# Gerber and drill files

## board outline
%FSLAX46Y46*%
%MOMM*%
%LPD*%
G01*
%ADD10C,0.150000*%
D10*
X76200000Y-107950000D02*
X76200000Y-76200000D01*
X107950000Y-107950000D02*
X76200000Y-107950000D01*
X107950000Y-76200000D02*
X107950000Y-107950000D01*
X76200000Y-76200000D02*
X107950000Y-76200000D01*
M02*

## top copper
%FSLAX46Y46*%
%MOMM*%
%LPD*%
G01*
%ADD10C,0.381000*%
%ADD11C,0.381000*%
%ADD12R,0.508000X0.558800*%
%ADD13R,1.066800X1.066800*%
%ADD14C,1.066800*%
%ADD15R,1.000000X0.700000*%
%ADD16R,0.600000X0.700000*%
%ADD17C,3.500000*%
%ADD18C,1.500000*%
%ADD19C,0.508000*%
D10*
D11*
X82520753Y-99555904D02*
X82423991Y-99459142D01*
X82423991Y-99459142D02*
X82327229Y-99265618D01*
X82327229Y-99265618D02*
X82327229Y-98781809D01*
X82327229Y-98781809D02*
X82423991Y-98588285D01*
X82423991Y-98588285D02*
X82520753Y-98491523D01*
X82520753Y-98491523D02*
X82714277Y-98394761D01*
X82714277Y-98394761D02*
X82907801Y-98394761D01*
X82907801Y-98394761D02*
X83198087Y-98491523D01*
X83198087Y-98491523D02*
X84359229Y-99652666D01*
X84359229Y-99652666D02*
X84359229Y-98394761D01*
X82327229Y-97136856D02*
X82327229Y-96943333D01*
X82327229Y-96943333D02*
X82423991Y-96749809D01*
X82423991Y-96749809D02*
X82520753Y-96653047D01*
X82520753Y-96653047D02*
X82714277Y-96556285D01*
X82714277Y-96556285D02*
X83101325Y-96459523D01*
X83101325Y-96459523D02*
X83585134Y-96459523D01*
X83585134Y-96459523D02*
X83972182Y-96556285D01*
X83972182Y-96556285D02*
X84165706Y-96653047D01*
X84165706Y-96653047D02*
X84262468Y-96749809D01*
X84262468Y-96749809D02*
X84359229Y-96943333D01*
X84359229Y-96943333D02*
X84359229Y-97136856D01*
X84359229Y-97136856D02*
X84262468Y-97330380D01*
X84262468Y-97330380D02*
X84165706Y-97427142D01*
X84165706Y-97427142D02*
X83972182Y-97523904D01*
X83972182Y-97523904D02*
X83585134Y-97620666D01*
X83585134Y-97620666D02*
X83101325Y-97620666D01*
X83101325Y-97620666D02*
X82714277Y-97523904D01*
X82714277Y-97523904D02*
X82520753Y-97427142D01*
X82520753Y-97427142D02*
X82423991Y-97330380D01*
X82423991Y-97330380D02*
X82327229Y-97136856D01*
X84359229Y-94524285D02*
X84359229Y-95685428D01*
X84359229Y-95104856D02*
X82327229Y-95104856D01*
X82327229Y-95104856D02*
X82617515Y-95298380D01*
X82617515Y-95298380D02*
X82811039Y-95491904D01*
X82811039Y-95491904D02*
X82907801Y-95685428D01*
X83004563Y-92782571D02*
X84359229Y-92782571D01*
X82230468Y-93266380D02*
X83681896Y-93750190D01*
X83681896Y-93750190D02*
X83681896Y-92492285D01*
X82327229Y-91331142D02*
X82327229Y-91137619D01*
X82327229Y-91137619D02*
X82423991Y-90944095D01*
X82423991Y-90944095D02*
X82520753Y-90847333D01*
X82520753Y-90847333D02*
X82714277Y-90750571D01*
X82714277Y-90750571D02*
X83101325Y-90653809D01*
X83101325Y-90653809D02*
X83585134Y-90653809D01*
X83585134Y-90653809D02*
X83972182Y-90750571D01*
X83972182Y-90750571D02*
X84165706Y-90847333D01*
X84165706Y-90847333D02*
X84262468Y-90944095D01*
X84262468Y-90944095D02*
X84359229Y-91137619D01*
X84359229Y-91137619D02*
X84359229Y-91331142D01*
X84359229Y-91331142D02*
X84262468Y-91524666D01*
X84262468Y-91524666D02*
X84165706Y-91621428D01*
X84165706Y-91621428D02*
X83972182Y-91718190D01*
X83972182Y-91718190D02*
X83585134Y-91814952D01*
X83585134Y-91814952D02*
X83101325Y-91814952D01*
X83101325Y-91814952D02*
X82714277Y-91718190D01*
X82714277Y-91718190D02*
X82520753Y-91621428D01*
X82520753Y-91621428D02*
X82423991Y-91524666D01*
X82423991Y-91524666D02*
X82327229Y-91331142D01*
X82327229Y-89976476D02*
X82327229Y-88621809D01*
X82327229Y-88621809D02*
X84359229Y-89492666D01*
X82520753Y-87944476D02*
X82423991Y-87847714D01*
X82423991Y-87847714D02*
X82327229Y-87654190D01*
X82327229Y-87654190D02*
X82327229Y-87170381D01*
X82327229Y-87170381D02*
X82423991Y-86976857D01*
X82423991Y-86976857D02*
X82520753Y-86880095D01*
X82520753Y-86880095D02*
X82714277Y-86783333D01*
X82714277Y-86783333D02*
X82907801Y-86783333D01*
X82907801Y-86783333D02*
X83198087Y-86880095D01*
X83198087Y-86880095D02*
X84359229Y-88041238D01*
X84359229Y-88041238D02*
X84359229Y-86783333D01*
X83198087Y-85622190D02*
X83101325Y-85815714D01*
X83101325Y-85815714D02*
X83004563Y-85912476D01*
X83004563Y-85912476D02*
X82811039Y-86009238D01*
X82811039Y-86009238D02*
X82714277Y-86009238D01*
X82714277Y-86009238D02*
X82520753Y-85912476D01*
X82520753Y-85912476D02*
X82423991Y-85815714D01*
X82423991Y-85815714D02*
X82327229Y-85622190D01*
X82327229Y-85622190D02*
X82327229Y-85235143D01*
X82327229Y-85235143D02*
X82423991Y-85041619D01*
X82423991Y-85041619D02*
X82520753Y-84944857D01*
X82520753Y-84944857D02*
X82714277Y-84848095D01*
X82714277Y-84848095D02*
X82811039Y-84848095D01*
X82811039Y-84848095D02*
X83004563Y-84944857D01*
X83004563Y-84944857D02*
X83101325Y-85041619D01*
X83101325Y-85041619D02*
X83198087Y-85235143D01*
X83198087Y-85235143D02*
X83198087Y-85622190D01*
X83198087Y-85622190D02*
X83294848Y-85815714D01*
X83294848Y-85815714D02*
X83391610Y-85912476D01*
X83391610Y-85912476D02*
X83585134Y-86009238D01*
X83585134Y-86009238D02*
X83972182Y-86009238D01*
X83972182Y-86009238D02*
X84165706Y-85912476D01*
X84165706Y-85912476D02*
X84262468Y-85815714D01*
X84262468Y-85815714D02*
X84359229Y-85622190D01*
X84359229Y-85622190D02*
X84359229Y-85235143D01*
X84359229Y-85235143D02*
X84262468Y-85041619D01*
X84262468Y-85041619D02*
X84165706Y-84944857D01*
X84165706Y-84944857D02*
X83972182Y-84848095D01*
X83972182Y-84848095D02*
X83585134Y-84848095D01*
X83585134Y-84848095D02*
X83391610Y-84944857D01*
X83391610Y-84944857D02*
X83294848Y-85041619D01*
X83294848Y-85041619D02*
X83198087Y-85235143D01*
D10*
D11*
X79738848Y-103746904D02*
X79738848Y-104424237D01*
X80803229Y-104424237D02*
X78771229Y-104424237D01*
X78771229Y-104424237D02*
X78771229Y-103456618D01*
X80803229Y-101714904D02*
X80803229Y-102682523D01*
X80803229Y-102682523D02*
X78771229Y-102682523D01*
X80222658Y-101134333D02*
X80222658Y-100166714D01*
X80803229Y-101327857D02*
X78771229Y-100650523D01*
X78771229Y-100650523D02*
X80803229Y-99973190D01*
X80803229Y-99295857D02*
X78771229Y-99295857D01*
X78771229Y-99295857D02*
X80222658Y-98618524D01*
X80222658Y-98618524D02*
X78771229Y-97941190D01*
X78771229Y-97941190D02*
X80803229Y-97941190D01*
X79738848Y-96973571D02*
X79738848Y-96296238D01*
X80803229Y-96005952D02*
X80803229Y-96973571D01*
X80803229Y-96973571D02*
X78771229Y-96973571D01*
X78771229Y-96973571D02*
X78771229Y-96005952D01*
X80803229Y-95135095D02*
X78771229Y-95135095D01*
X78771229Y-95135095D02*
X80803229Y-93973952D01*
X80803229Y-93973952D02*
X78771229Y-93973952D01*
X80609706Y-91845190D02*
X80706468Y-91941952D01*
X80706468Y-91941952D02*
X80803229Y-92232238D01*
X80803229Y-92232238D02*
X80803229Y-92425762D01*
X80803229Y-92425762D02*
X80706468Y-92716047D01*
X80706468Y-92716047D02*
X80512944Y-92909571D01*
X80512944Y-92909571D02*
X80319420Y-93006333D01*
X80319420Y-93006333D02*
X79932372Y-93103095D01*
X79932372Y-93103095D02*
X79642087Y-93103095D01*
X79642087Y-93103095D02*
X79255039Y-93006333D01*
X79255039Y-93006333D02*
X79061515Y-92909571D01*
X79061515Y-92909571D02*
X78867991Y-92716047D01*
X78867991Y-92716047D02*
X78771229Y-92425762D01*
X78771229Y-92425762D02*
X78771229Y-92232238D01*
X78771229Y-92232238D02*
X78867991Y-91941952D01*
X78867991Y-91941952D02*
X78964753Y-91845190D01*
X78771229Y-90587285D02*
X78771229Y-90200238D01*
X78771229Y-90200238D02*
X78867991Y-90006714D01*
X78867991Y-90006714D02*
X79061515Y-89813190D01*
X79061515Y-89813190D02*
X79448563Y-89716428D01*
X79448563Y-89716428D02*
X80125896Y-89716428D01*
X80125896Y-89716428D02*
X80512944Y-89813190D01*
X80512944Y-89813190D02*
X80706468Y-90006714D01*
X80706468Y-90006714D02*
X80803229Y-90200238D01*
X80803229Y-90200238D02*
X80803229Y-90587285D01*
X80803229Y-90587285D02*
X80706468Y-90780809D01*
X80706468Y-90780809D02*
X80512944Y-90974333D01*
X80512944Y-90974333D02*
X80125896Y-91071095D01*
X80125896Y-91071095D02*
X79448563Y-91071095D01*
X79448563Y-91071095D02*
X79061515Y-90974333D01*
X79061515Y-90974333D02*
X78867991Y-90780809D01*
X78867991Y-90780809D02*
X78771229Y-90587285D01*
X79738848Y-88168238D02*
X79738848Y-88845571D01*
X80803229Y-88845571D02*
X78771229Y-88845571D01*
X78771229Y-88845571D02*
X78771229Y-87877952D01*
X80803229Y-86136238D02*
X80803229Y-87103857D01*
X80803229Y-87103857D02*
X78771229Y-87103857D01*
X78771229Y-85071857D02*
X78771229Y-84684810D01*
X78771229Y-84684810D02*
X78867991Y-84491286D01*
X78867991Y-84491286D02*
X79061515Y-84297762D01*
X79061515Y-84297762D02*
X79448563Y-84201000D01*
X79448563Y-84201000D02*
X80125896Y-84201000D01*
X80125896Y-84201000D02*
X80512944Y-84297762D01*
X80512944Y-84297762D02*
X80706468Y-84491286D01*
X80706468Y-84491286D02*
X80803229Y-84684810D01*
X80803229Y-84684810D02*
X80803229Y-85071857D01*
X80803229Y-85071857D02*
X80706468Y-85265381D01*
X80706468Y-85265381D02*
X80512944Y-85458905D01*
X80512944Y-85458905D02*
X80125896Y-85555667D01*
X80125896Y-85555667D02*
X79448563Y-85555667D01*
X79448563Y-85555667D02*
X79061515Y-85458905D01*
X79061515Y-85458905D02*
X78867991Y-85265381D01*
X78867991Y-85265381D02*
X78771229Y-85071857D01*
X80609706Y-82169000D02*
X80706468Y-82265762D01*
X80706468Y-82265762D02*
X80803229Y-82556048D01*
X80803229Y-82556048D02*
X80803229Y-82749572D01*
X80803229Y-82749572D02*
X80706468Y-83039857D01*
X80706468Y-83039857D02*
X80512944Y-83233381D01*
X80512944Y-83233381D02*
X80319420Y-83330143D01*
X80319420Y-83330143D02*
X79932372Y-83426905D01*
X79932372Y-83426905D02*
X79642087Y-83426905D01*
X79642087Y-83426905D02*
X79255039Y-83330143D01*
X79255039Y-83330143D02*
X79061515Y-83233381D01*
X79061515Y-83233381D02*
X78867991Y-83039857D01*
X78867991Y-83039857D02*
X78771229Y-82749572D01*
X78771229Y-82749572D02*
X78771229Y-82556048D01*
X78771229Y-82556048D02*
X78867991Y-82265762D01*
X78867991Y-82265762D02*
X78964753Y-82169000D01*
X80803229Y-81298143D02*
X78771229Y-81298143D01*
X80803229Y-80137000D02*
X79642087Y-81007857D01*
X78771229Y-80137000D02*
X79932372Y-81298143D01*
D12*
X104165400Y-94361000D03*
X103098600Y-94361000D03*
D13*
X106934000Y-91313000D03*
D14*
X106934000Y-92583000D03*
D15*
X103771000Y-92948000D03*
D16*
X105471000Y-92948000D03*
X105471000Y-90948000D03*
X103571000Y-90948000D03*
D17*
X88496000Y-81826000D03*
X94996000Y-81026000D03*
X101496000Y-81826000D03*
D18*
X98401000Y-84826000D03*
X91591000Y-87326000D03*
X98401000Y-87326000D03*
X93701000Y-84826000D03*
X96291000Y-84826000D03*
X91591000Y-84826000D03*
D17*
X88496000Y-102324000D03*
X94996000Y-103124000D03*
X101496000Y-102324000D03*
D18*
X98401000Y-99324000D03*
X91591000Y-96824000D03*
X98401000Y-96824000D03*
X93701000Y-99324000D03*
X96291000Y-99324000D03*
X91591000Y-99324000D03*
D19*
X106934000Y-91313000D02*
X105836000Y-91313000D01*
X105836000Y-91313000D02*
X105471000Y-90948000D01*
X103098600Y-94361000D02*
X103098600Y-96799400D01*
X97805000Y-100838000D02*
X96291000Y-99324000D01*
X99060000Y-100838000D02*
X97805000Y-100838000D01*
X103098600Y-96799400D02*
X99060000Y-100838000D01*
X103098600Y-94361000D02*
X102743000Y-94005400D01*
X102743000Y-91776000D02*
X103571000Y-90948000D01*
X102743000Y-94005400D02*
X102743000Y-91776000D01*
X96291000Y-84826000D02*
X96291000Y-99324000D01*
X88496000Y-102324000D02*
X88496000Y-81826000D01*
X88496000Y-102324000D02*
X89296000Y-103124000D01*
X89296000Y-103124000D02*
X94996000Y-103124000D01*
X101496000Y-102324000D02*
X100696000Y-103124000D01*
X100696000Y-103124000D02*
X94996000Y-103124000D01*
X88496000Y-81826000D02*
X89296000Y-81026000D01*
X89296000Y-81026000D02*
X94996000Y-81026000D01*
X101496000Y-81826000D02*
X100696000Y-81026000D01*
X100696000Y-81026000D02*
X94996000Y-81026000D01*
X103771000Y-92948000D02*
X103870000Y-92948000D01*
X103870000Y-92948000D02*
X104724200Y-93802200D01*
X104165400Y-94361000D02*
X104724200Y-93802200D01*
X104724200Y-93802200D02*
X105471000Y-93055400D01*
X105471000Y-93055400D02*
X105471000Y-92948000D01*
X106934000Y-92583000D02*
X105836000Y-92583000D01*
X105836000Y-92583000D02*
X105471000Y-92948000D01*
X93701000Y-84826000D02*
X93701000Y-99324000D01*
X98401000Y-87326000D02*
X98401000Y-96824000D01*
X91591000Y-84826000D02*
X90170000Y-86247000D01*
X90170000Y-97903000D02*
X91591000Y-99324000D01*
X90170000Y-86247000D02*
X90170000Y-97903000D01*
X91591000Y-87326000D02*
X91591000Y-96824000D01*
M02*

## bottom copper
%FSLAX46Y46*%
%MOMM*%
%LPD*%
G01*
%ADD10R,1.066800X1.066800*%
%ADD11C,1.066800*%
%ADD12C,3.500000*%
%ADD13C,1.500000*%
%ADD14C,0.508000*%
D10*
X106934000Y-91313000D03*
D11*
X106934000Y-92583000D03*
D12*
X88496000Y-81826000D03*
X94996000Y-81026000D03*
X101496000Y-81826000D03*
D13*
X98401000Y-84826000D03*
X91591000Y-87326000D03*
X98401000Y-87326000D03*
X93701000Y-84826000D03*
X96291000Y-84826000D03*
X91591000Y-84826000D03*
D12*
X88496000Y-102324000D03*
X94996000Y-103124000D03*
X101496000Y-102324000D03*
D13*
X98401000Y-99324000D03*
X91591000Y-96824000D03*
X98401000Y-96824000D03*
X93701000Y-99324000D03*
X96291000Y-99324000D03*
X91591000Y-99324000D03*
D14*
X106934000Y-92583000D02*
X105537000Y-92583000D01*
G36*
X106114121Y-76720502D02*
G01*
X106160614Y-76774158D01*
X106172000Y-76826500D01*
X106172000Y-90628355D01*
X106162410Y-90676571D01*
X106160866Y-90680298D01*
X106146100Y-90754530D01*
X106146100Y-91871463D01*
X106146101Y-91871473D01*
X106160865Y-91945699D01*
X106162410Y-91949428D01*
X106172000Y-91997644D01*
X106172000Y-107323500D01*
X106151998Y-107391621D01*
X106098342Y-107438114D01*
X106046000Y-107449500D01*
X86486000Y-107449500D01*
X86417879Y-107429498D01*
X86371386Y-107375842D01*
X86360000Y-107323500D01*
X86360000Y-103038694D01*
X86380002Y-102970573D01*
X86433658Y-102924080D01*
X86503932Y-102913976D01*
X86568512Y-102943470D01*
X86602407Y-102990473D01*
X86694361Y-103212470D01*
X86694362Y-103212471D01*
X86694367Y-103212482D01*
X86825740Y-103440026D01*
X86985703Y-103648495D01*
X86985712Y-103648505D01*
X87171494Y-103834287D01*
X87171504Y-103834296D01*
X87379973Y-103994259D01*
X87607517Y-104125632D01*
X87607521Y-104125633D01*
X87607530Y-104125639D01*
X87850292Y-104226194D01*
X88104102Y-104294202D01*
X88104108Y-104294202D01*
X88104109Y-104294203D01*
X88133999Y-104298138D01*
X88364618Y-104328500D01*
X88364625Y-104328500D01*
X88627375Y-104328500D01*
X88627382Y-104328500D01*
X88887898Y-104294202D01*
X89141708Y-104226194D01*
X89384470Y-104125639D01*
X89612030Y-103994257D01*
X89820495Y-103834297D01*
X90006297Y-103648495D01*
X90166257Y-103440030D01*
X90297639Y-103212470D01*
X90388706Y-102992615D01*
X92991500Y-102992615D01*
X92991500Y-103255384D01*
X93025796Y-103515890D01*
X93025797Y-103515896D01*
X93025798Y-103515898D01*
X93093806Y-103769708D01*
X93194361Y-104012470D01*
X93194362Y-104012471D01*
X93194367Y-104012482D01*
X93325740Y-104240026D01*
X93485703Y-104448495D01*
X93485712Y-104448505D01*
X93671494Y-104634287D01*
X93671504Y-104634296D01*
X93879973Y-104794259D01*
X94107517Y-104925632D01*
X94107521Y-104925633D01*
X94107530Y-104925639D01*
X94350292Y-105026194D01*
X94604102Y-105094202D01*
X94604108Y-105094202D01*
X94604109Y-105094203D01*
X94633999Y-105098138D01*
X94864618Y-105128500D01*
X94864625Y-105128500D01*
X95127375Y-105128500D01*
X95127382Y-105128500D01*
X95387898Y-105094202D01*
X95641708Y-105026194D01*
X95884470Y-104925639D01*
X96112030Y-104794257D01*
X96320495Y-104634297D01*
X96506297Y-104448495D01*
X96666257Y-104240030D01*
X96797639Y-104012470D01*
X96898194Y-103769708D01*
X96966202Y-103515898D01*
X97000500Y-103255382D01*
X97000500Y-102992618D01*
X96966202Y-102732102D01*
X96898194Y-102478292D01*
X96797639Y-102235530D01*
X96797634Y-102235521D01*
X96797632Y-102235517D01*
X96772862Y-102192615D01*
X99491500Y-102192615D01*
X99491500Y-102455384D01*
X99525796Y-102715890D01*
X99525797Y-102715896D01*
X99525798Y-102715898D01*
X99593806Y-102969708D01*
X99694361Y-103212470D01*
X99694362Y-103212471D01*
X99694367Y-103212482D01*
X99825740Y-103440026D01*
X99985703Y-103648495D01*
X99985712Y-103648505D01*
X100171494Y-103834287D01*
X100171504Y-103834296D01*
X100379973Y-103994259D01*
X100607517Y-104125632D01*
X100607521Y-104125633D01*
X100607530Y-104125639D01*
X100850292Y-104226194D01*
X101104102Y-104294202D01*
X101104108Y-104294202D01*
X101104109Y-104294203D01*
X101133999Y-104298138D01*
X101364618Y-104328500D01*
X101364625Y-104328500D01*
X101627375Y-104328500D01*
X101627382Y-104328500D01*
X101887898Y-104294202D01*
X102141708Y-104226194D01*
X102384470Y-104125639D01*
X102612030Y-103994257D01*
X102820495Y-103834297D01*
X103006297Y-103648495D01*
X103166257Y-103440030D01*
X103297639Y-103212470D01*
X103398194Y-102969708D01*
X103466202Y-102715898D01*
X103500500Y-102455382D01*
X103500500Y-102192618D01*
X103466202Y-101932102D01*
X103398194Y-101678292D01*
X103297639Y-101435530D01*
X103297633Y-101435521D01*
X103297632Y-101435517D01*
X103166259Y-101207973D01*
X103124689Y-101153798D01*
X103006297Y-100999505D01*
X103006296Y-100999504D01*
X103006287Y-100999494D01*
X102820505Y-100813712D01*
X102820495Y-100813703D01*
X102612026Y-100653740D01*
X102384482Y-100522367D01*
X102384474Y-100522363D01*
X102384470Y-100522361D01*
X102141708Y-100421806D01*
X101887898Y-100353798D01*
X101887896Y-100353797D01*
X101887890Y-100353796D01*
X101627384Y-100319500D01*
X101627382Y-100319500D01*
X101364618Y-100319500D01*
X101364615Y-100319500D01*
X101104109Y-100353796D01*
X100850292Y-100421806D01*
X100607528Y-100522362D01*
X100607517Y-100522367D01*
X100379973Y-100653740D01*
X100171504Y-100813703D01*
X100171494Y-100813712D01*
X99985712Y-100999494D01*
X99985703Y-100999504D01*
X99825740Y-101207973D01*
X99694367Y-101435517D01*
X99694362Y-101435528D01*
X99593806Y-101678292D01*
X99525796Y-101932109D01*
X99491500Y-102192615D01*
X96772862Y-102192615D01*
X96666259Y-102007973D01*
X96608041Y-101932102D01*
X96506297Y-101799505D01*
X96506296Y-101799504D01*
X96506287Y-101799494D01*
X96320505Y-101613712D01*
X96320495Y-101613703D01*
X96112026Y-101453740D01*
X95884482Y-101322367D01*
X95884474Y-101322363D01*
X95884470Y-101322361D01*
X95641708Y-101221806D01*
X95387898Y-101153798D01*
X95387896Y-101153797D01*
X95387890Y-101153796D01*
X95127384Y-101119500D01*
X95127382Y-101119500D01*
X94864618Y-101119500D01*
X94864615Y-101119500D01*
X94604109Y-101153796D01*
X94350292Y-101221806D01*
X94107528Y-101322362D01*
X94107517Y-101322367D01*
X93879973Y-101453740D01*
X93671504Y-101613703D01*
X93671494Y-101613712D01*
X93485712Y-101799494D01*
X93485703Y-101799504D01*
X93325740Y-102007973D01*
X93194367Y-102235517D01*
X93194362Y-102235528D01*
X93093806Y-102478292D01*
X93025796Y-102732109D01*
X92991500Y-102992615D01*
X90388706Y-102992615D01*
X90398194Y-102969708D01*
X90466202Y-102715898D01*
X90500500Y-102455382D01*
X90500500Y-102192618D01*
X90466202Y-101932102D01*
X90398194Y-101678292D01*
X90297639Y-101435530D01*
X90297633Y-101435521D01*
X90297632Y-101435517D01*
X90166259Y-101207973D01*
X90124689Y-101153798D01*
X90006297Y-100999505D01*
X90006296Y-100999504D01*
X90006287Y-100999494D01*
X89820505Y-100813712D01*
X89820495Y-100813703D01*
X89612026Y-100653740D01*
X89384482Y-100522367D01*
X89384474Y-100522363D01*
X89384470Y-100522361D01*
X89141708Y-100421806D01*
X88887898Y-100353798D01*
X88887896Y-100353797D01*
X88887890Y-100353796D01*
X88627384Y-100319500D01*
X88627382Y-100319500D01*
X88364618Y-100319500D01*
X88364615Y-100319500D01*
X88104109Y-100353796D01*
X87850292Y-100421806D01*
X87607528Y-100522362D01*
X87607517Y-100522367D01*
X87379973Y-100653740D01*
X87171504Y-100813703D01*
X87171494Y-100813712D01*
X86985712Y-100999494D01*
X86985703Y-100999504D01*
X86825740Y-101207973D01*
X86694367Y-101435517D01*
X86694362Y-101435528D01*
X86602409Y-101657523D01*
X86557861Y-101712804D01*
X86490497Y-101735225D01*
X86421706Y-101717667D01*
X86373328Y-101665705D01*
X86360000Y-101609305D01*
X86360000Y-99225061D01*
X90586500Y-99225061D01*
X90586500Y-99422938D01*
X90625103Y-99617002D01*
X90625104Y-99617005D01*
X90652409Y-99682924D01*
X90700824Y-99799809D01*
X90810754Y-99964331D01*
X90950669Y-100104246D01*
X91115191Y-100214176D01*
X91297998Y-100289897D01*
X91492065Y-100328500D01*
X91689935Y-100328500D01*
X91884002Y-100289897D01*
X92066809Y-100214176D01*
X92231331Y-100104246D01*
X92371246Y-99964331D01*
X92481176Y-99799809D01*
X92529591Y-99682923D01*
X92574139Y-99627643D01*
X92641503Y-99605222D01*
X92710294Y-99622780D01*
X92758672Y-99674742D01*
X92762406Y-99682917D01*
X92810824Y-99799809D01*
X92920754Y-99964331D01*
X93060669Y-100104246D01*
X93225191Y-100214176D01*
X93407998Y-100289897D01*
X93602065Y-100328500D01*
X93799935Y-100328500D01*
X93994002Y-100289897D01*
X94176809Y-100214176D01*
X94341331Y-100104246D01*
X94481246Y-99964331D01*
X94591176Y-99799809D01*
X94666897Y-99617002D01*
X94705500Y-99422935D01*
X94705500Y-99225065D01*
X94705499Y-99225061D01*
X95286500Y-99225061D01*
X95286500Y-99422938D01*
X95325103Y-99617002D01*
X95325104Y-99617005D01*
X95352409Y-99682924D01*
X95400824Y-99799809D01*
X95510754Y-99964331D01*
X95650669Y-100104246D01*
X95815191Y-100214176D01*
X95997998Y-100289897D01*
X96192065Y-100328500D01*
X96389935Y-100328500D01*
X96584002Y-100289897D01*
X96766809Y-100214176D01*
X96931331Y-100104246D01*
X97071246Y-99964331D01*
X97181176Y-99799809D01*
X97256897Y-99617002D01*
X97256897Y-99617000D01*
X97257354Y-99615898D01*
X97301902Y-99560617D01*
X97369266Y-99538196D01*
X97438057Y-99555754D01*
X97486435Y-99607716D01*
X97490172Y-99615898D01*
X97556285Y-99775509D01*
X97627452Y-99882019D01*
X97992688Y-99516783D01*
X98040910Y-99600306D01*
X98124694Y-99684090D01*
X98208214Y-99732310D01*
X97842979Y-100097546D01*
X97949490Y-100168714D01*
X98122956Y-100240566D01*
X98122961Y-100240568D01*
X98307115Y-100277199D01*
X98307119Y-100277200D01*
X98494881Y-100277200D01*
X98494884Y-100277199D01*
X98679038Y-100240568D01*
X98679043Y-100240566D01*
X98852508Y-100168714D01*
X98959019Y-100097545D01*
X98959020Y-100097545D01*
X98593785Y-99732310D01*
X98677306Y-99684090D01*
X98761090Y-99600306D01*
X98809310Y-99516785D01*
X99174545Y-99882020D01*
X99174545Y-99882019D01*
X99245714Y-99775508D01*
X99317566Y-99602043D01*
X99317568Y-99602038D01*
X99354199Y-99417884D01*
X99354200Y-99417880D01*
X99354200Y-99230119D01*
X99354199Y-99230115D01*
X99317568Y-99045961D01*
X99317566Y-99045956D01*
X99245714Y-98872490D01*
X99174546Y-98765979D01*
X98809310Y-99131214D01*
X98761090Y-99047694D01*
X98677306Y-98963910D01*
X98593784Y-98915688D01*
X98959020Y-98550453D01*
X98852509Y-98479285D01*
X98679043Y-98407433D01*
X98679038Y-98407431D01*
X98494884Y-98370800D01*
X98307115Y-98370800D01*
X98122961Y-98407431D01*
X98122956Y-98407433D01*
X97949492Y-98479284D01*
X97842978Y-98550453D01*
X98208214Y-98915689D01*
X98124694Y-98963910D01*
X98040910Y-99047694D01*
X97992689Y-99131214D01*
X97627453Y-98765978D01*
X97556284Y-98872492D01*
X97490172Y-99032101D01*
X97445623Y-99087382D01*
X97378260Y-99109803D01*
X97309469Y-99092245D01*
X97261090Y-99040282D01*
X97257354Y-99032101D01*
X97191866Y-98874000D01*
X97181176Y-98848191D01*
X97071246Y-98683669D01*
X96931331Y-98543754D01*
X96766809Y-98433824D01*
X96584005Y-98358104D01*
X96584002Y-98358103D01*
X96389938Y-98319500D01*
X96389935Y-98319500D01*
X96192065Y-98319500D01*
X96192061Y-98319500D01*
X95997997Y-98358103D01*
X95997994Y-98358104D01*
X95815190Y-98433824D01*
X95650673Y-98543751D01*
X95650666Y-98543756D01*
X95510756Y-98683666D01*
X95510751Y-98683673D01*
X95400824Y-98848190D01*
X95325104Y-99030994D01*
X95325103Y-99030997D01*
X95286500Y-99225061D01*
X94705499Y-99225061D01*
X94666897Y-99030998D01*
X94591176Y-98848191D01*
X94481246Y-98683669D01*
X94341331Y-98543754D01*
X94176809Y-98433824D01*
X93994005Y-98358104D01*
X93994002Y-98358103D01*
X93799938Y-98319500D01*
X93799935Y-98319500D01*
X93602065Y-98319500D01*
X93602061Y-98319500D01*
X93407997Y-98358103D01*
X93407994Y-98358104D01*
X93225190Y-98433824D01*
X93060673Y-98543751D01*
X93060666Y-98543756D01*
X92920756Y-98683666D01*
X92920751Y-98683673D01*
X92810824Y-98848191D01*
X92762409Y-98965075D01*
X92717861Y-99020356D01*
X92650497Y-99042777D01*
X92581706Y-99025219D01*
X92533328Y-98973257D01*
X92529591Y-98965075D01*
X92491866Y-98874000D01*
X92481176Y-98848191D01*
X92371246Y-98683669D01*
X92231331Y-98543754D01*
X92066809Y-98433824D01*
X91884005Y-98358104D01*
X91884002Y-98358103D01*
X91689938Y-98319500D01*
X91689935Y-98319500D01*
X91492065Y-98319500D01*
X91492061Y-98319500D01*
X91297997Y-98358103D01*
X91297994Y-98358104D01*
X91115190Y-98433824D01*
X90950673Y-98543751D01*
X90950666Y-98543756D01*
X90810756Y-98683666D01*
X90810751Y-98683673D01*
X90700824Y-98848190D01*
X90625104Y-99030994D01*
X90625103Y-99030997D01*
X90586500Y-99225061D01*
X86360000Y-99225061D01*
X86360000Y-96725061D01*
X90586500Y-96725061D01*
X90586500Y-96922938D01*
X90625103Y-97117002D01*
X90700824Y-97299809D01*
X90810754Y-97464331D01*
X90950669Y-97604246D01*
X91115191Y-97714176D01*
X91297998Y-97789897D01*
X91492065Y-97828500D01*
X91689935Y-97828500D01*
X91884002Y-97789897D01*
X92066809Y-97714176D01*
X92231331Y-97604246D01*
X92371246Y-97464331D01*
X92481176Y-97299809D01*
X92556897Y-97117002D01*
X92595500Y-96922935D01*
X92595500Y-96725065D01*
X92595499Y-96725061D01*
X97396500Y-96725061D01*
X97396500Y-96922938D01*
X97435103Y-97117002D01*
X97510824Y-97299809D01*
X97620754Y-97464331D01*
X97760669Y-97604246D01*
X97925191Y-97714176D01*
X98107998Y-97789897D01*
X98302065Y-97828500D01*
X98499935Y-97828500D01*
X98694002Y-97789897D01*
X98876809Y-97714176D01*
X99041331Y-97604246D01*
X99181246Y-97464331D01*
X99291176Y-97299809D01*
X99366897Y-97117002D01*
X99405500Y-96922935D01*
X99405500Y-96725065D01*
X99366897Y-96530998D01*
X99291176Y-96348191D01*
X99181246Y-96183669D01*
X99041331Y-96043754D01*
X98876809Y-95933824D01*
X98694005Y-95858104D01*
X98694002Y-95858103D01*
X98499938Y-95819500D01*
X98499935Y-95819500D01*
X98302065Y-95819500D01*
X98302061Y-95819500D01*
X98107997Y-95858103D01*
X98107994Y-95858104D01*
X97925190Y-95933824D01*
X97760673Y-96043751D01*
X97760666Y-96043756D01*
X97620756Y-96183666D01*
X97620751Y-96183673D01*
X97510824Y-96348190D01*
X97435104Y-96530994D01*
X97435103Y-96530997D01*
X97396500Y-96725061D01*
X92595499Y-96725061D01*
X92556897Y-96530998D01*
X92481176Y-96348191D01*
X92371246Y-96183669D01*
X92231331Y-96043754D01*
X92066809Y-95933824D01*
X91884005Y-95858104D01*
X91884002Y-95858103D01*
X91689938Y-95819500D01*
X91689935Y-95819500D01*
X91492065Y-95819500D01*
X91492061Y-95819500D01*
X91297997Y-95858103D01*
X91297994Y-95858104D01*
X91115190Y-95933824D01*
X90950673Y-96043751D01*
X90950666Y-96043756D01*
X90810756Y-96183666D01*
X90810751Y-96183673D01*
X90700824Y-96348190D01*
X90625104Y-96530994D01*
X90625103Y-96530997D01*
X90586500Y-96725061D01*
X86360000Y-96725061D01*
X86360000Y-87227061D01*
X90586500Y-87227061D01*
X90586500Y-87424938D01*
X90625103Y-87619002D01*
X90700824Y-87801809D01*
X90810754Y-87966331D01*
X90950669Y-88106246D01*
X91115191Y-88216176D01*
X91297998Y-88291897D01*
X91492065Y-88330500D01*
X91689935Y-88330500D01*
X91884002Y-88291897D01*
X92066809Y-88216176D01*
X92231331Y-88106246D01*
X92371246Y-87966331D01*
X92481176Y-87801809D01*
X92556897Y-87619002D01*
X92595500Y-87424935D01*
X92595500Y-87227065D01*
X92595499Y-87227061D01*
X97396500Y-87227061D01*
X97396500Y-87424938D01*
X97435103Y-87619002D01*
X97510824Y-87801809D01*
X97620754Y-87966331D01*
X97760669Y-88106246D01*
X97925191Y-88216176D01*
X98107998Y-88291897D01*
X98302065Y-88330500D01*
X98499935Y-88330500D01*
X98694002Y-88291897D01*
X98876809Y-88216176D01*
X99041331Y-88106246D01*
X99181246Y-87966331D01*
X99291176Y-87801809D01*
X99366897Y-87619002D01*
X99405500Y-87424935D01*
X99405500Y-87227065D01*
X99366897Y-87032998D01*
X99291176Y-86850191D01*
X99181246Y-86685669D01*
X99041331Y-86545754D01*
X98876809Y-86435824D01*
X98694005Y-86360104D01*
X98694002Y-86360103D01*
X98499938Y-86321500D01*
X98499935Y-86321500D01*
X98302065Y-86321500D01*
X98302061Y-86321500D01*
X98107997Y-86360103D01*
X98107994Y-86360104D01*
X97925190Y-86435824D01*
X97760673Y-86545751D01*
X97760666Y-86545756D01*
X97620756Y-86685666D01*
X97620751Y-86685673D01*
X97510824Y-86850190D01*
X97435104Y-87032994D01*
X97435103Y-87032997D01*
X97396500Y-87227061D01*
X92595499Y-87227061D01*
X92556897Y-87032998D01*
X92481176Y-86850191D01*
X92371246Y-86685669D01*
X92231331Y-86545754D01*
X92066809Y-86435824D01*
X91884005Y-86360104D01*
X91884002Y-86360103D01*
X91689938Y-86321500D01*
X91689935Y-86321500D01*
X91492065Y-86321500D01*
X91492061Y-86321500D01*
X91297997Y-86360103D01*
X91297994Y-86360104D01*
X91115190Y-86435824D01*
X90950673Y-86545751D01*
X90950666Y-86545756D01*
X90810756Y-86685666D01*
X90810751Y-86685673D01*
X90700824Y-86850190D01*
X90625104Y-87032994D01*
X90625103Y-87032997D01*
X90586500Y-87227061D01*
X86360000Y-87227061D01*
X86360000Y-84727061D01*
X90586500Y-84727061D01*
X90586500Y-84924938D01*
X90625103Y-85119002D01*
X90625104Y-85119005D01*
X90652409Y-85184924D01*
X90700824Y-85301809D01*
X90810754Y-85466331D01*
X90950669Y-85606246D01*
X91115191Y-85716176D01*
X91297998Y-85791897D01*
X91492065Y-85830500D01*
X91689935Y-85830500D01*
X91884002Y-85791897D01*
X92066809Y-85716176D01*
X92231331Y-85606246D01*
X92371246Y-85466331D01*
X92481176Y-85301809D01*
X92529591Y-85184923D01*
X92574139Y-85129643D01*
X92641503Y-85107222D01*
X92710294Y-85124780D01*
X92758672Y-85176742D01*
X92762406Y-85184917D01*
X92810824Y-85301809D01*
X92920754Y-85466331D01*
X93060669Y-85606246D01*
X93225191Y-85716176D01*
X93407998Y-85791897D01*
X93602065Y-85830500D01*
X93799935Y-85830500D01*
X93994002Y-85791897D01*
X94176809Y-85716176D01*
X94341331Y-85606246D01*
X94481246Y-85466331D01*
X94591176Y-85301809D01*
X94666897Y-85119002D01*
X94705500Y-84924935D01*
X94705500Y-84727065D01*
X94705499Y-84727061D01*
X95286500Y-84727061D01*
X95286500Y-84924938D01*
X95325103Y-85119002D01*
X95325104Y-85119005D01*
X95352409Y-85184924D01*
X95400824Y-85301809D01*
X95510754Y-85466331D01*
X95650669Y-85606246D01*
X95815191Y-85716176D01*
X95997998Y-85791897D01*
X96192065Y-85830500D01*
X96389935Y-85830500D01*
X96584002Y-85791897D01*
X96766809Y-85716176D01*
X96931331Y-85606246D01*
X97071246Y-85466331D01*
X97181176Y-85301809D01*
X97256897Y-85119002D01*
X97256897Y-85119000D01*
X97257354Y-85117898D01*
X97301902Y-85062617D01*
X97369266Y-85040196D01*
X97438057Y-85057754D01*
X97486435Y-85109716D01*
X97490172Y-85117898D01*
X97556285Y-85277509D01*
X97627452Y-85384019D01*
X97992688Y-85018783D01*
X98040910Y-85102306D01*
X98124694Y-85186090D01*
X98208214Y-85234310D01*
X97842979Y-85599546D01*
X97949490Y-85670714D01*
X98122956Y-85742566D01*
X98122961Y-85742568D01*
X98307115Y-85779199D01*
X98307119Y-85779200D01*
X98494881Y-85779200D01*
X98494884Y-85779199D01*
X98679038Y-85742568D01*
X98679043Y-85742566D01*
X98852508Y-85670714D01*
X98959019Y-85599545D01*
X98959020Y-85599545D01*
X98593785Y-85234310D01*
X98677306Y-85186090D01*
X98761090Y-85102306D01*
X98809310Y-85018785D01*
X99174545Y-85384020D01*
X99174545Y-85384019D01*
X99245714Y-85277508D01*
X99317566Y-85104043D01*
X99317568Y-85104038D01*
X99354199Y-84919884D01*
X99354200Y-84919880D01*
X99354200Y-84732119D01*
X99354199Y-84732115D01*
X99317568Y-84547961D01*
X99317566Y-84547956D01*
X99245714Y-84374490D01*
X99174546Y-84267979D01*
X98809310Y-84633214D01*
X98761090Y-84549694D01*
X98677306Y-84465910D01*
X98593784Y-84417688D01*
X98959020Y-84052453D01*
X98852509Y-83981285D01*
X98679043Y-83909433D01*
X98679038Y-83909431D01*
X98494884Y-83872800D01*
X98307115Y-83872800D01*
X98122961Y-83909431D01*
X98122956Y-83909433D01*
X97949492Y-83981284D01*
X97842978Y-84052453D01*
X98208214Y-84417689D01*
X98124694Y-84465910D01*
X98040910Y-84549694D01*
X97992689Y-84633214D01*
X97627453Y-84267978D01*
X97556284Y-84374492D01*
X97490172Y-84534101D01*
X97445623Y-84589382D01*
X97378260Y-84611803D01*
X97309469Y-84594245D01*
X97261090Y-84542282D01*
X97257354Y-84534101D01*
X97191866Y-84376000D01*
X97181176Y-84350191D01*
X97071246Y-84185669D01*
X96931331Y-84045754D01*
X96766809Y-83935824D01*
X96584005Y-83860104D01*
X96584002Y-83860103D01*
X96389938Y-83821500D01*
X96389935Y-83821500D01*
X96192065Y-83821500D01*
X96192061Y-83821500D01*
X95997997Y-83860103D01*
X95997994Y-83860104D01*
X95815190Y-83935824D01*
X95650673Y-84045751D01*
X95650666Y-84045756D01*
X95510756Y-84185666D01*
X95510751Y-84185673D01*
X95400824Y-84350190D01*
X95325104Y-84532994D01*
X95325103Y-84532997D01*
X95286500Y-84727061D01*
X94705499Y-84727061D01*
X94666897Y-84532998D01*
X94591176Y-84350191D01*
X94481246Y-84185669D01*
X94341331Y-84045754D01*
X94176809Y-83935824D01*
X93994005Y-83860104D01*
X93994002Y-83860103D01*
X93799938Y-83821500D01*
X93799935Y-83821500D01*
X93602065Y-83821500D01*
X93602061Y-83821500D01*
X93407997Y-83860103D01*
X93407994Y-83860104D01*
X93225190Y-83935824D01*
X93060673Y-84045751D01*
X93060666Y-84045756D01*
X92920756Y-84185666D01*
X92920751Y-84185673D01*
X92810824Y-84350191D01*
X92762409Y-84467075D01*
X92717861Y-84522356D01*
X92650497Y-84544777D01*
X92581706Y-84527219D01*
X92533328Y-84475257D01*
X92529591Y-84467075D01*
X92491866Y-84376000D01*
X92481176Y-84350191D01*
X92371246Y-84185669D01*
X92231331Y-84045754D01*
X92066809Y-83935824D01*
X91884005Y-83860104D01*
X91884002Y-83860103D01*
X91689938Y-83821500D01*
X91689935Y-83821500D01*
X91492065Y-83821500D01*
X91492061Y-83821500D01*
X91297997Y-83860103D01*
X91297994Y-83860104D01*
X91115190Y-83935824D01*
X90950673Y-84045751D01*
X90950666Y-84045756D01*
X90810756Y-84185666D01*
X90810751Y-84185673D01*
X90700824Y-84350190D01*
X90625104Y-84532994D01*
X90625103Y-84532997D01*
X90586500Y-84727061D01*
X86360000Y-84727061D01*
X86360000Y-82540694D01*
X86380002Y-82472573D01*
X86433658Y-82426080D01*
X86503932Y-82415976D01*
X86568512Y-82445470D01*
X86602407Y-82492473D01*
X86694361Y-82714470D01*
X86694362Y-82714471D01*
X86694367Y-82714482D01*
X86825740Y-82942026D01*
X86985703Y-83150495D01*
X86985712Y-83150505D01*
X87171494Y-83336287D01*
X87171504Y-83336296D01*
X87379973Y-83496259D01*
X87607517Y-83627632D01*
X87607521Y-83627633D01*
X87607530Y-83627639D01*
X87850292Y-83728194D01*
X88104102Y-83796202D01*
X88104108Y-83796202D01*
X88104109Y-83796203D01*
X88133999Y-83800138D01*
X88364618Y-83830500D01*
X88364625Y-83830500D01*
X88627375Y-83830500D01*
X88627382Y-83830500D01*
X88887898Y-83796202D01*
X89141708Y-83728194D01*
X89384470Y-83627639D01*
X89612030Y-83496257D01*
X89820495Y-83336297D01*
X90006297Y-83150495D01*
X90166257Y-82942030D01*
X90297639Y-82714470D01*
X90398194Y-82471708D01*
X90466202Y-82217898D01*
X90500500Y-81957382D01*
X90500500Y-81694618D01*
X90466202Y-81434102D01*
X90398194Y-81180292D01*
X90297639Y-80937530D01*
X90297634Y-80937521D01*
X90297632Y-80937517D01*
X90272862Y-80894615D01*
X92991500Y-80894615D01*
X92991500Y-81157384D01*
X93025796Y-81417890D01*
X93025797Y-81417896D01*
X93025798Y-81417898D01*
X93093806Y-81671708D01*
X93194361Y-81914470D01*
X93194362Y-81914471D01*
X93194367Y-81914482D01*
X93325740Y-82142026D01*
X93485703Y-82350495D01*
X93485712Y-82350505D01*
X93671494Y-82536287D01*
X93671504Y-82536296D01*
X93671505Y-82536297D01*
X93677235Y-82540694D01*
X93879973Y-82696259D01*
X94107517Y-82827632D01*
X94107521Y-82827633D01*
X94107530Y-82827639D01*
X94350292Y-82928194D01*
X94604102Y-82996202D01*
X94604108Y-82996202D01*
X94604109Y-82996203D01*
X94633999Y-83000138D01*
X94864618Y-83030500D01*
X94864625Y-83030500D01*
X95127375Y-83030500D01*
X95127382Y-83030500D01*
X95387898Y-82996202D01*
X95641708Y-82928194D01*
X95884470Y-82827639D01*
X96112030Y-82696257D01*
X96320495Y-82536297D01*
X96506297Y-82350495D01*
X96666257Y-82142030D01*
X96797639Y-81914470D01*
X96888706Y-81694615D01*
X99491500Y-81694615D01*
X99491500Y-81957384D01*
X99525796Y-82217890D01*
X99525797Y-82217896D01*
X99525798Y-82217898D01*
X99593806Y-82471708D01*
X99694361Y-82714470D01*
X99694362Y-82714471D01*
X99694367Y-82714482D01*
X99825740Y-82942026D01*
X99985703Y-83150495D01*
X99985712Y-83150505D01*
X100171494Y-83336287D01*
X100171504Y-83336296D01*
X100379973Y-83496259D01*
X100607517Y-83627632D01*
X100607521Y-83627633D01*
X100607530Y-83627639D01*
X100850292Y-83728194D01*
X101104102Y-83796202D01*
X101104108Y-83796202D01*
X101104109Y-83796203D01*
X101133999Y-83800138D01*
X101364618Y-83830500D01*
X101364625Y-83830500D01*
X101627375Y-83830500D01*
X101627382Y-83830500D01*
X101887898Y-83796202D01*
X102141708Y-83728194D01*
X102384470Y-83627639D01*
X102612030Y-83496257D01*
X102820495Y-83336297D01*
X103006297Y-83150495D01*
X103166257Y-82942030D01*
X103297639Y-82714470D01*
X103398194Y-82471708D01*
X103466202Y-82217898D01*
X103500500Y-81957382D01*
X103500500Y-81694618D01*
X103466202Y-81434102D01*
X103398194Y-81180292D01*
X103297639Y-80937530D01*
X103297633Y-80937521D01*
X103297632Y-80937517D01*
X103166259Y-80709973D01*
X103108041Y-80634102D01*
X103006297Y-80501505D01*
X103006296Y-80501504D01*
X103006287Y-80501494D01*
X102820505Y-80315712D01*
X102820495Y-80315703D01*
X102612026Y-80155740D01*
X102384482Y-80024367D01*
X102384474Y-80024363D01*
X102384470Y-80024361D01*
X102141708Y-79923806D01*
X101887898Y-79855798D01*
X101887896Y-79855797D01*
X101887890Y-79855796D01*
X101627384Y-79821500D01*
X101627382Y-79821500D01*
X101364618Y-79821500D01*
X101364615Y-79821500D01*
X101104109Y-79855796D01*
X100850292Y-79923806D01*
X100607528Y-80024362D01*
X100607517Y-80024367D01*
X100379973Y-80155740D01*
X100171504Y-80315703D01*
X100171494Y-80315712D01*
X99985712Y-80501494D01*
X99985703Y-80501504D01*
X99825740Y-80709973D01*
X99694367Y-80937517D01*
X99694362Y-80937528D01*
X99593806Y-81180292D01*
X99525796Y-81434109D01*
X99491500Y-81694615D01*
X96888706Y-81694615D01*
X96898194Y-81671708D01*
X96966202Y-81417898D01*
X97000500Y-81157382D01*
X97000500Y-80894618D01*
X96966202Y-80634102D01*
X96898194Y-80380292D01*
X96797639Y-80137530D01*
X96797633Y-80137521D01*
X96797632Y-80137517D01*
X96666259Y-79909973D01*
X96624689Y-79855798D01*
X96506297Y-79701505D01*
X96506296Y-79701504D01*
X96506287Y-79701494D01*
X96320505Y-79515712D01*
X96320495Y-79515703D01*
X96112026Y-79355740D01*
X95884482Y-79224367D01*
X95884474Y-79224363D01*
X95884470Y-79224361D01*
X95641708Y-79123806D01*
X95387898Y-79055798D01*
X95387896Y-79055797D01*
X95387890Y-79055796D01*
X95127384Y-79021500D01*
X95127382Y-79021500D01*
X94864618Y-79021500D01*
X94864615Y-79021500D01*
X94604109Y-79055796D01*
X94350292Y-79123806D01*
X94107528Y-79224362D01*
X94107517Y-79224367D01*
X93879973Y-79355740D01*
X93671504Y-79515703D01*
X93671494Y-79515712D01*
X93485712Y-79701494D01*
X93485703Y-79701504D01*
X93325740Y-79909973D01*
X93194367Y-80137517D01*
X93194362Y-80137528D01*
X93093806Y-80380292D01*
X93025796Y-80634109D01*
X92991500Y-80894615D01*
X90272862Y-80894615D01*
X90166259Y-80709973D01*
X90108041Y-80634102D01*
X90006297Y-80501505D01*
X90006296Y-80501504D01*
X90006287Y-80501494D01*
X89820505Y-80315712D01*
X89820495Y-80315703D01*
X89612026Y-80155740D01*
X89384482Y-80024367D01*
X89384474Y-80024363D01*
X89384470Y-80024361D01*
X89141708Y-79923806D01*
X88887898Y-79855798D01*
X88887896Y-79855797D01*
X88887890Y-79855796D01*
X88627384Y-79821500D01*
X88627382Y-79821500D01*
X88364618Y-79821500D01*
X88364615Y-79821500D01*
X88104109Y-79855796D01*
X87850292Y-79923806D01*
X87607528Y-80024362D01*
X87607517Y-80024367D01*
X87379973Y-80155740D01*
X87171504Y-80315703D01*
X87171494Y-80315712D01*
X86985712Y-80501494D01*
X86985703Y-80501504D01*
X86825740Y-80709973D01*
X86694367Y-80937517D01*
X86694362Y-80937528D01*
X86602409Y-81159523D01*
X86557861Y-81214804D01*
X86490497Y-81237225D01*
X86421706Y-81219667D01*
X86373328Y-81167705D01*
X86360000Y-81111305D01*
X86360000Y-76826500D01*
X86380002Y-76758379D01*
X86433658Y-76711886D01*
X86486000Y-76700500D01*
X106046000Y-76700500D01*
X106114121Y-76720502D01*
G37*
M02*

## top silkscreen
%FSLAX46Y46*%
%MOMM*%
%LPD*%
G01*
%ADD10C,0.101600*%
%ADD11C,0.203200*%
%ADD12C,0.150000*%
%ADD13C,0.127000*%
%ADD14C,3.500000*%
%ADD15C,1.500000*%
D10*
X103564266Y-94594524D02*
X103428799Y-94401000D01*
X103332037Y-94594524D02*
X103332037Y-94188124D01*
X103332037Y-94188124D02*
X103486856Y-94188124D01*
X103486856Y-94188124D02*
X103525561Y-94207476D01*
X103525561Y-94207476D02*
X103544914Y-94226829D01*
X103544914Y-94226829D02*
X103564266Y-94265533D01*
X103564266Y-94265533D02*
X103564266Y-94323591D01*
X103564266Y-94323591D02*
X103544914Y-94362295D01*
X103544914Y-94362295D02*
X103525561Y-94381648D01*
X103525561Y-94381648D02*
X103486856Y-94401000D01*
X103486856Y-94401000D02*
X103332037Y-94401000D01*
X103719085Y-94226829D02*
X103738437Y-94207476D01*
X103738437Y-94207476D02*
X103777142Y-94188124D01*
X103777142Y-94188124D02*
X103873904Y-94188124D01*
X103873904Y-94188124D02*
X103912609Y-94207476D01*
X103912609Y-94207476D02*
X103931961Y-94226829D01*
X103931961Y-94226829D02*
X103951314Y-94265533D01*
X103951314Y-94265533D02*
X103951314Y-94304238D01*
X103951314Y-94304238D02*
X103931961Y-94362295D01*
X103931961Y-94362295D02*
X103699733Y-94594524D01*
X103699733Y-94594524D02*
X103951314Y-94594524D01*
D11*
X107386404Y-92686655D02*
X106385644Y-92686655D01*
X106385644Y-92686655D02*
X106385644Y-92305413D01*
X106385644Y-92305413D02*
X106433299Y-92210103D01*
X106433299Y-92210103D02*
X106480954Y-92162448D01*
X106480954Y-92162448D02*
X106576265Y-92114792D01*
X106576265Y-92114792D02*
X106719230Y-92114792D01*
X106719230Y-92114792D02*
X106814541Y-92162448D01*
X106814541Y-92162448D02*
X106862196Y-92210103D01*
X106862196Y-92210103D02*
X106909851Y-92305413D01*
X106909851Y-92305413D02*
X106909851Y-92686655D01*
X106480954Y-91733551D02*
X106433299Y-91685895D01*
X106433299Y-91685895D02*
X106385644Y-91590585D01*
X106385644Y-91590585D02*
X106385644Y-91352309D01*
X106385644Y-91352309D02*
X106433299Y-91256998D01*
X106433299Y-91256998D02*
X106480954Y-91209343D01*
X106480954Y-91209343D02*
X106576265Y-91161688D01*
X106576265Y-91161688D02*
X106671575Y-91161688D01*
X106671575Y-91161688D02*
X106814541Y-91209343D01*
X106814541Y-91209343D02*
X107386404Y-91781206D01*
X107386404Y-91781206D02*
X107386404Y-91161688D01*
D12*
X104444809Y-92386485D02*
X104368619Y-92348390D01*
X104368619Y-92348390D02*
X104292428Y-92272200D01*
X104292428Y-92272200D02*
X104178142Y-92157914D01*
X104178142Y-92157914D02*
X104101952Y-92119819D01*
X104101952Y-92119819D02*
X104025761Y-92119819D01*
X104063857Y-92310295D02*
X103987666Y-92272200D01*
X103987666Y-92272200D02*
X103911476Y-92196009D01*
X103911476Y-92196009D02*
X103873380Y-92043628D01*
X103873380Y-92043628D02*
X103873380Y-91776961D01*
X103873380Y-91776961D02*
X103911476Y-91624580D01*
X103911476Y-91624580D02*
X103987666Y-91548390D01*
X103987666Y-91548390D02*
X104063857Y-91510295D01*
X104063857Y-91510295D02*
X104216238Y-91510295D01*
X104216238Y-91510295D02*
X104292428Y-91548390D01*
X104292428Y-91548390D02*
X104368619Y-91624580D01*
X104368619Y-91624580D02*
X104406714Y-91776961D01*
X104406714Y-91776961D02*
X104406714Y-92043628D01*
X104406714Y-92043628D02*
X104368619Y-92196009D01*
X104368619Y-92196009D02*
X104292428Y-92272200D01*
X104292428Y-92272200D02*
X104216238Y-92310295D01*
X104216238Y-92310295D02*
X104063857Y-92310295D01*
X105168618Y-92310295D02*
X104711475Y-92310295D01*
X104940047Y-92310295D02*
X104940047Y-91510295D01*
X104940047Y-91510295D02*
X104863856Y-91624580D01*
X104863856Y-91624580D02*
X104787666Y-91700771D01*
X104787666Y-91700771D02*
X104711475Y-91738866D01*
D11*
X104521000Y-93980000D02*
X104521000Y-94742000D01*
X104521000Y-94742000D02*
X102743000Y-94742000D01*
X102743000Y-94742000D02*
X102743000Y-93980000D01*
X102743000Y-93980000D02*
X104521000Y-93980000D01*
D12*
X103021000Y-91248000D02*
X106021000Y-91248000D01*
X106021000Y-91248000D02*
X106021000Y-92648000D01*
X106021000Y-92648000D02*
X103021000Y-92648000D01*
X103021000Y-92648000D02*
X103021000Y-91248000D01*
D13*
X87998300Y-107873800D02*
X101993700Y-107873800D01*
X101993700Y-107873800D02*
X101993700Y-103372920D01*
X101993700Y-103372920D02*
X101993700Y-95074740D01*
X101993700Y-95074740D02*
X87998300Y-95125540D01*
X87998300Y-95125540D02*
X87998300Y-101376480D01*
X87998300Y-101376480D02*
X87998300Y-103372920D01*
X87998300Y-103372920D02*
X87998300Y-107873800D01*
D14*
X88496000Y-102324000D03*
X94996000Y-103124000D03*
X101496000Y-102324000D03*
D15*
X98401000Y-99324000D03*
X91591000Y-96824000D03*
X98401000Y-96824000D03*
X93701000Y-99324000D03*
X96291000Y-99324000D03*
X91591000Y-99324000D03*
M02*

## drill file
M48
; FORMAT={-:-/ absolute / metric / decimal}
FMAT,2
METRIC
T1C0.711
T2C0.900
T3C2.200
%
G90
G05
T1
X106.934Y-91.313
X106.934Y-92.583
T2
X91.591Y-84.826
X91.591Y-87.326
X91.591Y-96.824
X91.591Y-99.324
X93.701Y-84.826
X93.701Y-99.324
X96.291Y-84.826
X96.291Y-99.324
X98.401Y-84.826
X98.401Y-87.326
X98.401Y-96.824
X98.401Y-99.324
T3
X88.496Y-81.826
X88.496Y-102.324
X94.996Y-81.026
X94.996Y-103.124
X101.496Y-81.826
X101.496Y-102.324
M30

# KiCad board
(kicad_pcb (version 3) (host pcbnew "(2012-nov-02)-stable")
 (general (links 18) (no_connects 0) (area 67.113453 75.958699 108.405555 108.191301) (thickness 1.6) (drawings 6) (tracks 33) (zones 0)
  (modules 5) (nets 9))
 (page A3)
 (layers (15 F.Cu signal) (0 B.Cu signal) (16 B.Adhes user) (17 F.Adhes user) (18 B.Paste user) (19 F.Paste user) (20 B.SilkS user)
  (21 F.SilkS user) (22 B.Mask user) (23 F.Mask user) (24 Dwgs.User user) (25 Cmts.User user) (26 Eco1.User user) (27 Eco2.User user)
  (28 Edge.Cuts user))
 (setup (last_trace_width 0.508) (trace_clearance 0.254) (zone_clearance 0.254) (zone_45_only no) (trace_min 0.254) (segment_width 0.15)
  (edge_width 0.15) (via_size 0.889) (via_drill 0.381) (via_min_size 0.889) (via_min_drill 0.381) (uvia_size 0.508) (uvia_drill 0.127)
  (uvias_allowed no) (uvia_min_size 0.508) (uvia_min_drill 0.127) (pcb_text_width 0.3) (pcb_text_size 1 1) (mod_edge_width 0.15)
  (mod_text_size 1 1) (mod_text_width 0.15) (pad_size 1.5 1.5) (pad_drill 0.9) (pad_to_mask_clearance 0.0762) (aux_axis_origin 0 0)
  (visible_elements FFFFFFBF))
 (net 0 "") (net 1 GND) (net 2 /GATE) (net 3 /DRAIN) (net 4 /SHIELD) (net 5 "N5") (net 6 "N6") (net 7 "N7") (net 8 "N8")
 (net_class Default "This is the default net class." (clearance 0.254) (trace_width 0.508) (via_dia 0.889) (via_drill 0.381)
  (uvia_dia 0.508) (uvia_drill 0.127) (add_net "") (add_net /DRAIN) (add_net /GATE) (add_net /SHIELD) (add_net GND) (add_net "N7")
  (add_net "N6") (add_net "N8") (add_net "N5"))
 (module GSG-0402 (layer F.Cu) (at 103.632 94.361) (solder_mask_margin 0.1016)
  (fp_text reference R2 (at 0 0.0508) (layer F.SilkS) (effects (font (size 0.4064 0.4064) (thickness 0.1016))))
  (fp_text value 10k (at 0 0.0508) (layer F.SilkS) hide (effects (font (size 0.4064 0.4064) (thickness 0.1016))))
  (fp_line (start 0.889 -0.381) (end 0.889 0.381) (layer F.SilkS) (width 0.2032))
  (fp_line (start 0.889 0.381) (end -0.889 0.381) (layer F.SilkS) (width 0.2032))
  (fp_line (start -0.889 0.381) (end -0.889 -0.381) (layer F.SilkS) (width 0.2032))
  (fp_line (start -0.889 -0.381) (end 0.889 -0.381) (layer F.SilkS) (width 0.2032))
  (pad 2 smd rect (at 0.5334 0) (size 0.508 0.5588) (layers F.Cu F.Paste F.Mask) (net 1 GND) (solder_mask_margin 0.1016))
  (pad 1 smd rect (at -0.5334 0) (size 0.508 0.5588) (layers F.Cu F.Paste F.Mask) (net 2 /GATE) (die_length -2147.483648)
   (solder_mask_margin 0.1016)))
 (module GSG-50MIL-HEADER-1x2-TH (layer F.Cu) (at 106.934 91.948 270)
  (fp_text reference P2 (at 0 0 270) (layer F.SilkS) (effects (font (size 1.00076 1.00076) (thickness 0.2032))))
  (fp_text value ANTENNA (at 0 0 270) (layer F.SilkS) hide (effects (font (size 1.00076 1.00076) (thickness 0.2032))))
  (pad 1 thru_hole rect (at -0.635 0 270) (size 1.0668 1.0668) (drill 0.7112) (layers *.Cu *.Mask) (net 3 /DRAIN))
  (pad 2 thru_hole circle (at 0.635 0 270) (size 1.0668 1.0668) (drill 0.7112) (layers *.Cu *.Mask) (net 1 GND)))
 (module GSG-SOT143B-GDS (layer F.Cu) (at 104.521 91.948)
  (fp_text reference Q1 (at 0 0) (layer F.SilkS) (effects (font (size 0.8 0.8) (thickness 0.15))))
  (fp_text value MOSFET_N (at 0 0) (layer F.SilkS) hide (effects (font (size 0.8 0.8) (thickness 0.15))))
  (fp_line (start -1.5 -0.7) (end 1.5 -0.7) (layer F.SilkS) (width 0.15))
  (fp_line (start 1.5 -0.7) (end 1.5 0.7) (layer F.SilkS) (width 0.15))
  (fp_line (start 1.5 0.7) (end -1.5 0.7) (layer F.SilkS) (width 0.15))
  (fp_line (start -1.5 0.7) (end -1.5 -0.7) (layer F.SilkS) (width 0.15))
  (pad B smd rect (at -0.75 1) (size 1 0.7) (layers F.Cu F.Paste F.Mask) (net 1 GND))
  (pad S smd rect (at 0.95 1) (size 0.6 0.7) (layers F.Cu F.Paste F.Mask) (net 1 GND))
  (pad D smd rect (at 0.95 -1) (size 0.6 0.7) (layers F.Cu F.Paste F.Mask) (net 3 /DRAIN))
  (pad G smd rect (at -0.95 -1) (size 0.6 0.7) (layers F.Cu F.Paste F.Mask) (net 2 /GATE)))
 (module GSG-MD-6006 (layer B.Cu) (at 94.996 81.026 180)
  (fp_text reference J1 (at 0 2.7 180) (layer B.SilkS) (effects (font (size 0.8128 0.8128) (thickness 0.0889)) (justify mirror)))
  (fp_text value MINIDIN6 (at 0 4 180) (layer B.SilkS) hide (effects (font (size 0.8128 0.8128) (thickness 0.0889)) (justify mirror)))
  (pad 0 thru_hole circle (at 6.5 -0.8 180) (size 3.5 3.5) (drill 2.2) (layers *.Cu *.Mask B.SilkS) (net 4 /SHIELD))
  (pad 0 thru_hole circle (at 0 0 180) (size 3.5 3.5) (drill 2.2) (layers *.Cu *.Mask B.SilkS) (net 4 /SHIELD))
  (pad 0 thru_hole circle (at -6.5 -0.8 180) (size 3.5 3.5) (drill 2.2) (layers *.Cu *.Mask B.SilkS) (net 4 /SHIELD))
  (pad 3 thru_hole circle (at -3.405 -3.8 180) (size 1.5 1.5) (drill 0.9) (layers *.Cu *.Mask B.SilkS) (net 1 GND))
  (pad 6 thru_hole circle (at 3.405 -6.3 180) (size 1.5 1.5) (drill 0.9) (layers *.Cu *.Mask B.SilkS) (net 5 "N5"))
  (pad 5 thru_hole circle (at -3.405 -6.3 180) (size 1.5 1.5) (drill 0.9) (layers *.Cu *.Mask B.SilkS) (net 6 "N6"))
  (pad 2 thru_hole circle (at 1.295 -3.8 180) (size 1.5 1.5) (drill 0.9) (layers *.Cu *.Mask B.SilkS) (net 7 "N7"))
  (pad 1 thru_hole circle (at -1.295 -3.8 180) (size 1.5 1.5) (drill 0.9) (layers *.Cu *.Mask B.SilkS) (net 2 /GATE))
  (pad 4 thru_hole circle (at 3.405 -3.8 180) (size 1.5 1.5) (drill 0.9) (layers *.Cu *.Mask B.SilkS) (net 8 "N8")))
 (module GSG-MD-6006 (layer F.Cu) (at 94.996 103.124 180)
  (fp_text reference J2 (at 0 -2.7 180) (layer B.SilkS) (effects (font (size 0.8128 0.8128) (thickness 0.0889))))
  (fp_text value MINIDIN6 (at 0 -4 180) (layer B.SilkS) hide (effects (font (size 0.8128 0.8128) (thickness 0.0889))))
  (fp_line (start 6.9977 -4.7498) (end -6.9977 -4.7498) (layer F.SilkS) (width 0.127))
  (fp_line (start -6.9977 -4.7498) (end -6.9977 -0.24892) (layer F.SilkS) (width 0.127))
  (fp_line (start -6.9977 -0.24892) (end -6.9977 8.04926) (layer F.SilkS) (width 0.127))
  (fp_line (start -6.9977 8.04926) (end 6.9977 7.99846) (layer F.SilkS) (width 0.127))
  (fp_line (start 6.9977 7.99846) (end 6.9977 1.74752) (layer F.SilkS) (width 0.127))
  (fp_line (start 6.9977 1.74752) (end 6.9977 -0.24892) (layer F.SilkS) (width 0.127))
  (fp_line (start 6.9977 -0.24892) (end 6.9977 -4.7498) (layer F.SilkS) (width 0.127))
  (pad 0 thru_hole circle (at 6.5 0.8 180) (size 3.5 3.5) (drill 2.2) (layers *.Cu *.Mask F.SilkS) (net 4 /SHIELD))
  (pad 0 thru_hole circle (at 0 0 180) (size 3.5 3.5) (drill 2.2) (layers *.Cu *.Mask F.SilkS) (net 4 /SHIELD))
  (pad 0 thru_hole circle (at -6.5 0.8 180) (size 3.5 3.5) (drill 2.2) (layers *.Cu *.Mask F.SilkS) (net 4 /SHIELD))
  (pad 3 thru_hole circle (at -3.405 3.8 180) (size 1.5 1.5) (drill 0.9) (layers *.Cu *.Mask F.SilkS) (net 1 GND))
  (pad 6 thru_hole circle (at 3.405 6.3 180) (size 1.5 1.5) (drill 0.9) (layers *.Cu *.Mask F.SilkS) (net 5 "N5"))
  (pad 5 thru_hole circle (at -3.405 6.3 180) (size 1.5 1.5) (drill 0.9) (layers *.Cu *.Mask F.SilkS) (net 6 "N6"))
  (pad 2 thru_hole circle (at 1.295 3.8 180) (size 1.5 1.5) (drill 0.9) (layers *.Cu *.Mask F.SilkS) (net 7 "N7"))
  (pad 1 thru_hole circle (at -1.295 3.8 180) (size 1.5 1.5) (drill 0.9) (layers *.Cu *.Mask F.SilkS) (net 2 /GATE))
  (pad 4 thru_hole circle (at 3.405 3.8 180) (size 1.5 1.5) (drill 0.9) (layers *.Cu *.Mask F.SilkS) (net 8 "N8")))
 (gr_line (start 76.2 107.95) (end 76.2 76.2) (angle 90) (layer Edge.Cuts) (width 0.15))
 (gr_line (start 107.95 107.95) (end 76.2 107.95) (angle 90) (layer Edge.Cuts) (width 0.15))
 (gr_line (start 107.95 76.2) (end 107.95 107.95) (angle 90) (layer Edge.Cuts) (width 0.15))
 (gr_line (start 76.2 76.2) (end 107.95 76.2) (angle 90) (layer Edge.Cuts) (width 0.15))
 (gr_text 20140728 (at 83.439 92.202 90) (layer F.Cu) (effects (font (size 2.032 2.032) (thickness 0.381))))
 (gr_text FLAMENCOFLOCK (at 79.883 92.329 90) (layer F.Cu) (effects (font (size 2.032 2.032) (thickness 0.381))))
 (segment (start 106.934 91.313) (end 105.836 91.313) (width 0.508) (layer F.Cu) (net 3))
 (segment (start 105.836 91.313) (end 105.471 90.948) (width 0.508) (layer F.Cu) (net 3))
 (segment (start 103.0986 94.361) (end 103.0986 96.7994) (width 0.508) (layer F.Cu) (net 2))
 (segment (start 97.805 100.838) (end 96.291 99.324) (width 0.508) (layer F.Cu) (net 2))
 (segment (start 99.06 100.838) (end 97.805 100.838) (width 0.508) (layer F.Cu) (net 2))
 (segment (start 103.0986 96.7994) (end 99.06 100.838) (width 0.508) (layer F.Cu) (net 2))
 (segment (start 103.0986 94.361) (end 102.743 94.0054) (width 0.508) (layer F.Cu) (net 2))
 (segment (start 102.743 91.776) (end 103.571 90.948) (width 0.508) (layer F.Cu) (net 2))
 (segment (start 102.743 94.0054) (end 102.743 91.776) (width 0.508) (layer F.Cu) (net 2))
 (segment (start 96.291 84.826) (end 96.291 99.324) (width 0.508) (layer F.Cu) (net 2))
 (segment (start 88.496 102.324) (end 88.496 81.826) (width 0.508) (layer F.Cu) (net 4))
 (segment (start 88.496 102.324) (end 89.296 103.124) (width 0.508) (layer F.Cu) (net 4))
 (segment (start 89.296 103.124) (end 94.996 103.124) (width 0.508) (layer F.Cu) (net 4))
 (segment (start 101.496 102.324) (end 100.696 103.124) (width 0.508) (layer F.Cu) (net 4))
 (segment (start 100.696 103.124) (end 94.996 103.124) (width 0.508) (layer F.Cu) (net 4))
 (segment (start 88.496 81.826) (end 89.296 81.026) (width 0.508) (layer F.Cu) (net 4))
 (segment (start 89.296 81.026) (end 94.996 81.026) (width 0.508) (layer F.Cu) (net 4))
 (segment (start 101.496 81.826) (end 100.696 81.026) (width 0.508) (layer F.Cu) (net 4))
 (segment (start 100.696 81.026) (end 94.996 81.026) (width 0.508) (layer F.Cu) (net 4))
 (segment (start 103.771 92.948) (end 103.87 92.948) (width 0.508) (layer F.Cu) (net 1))
 (segment (start 103.87 92.948) (end 104.7242 93.8022) (width 0.508) (layer F.Cu) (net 1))
 (segment (start 104.1654 94.361) (end 104.7242 93.8022) (width 0.508) (layer F.Cu) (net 1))
 (segment (start 104.7242 93.8022) (end 105.471 93.0554) (width 0.508) (layer F.Cu) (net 1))
 (segment (start 105.471 93.0554) (end 105.471 92.948) (width 0.508) (layer F.Cu) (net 1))
 (segment (start 106.934 92.583) (end 105.836 92.583) (width 0.508) (layer F.Cu) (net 1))
 (segment (start 105.836 92.583) (end 105.471 92.948) (width 0.508) (layer F.Cu) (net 1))
 (segment (start 106.934 92.583) (end 105.537 92.583) (width 0.508) (layer B.Cu) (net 1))
 (segment (start 93.701 84.826) (end 93.701 99.324) (width 0.508) (layer F.Cu) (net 7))
 (segment (start 98.401 87.326) (end 98.401 96.824) (width 0.508) (layer F.Cu) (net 6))
 (segment (start 91.591 84.826) (end 90.17 86.247) (width 0.508) (layer F.Cu) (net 8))
 (segment (start 90.17 97.903) (end 91.591 99.324) (width 0.508) (layer F.Cu) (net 8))
 (segment (start 90.17 86.247) (end 90.17 97.903) (width 0.508) (layer F.Cu) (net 8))
 (segment (start 91.591 87.326) (end 91.591 96.824) (width 0.508) (layer F.Cu) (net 5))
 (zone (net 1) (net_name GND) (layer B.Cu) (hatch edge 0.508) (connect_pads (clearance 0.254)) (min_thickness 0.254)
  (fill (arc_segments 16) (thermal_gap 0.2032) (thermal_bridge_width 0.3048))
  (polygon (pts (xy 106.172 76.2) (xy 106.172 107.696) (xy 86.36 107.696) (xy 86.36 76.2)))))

